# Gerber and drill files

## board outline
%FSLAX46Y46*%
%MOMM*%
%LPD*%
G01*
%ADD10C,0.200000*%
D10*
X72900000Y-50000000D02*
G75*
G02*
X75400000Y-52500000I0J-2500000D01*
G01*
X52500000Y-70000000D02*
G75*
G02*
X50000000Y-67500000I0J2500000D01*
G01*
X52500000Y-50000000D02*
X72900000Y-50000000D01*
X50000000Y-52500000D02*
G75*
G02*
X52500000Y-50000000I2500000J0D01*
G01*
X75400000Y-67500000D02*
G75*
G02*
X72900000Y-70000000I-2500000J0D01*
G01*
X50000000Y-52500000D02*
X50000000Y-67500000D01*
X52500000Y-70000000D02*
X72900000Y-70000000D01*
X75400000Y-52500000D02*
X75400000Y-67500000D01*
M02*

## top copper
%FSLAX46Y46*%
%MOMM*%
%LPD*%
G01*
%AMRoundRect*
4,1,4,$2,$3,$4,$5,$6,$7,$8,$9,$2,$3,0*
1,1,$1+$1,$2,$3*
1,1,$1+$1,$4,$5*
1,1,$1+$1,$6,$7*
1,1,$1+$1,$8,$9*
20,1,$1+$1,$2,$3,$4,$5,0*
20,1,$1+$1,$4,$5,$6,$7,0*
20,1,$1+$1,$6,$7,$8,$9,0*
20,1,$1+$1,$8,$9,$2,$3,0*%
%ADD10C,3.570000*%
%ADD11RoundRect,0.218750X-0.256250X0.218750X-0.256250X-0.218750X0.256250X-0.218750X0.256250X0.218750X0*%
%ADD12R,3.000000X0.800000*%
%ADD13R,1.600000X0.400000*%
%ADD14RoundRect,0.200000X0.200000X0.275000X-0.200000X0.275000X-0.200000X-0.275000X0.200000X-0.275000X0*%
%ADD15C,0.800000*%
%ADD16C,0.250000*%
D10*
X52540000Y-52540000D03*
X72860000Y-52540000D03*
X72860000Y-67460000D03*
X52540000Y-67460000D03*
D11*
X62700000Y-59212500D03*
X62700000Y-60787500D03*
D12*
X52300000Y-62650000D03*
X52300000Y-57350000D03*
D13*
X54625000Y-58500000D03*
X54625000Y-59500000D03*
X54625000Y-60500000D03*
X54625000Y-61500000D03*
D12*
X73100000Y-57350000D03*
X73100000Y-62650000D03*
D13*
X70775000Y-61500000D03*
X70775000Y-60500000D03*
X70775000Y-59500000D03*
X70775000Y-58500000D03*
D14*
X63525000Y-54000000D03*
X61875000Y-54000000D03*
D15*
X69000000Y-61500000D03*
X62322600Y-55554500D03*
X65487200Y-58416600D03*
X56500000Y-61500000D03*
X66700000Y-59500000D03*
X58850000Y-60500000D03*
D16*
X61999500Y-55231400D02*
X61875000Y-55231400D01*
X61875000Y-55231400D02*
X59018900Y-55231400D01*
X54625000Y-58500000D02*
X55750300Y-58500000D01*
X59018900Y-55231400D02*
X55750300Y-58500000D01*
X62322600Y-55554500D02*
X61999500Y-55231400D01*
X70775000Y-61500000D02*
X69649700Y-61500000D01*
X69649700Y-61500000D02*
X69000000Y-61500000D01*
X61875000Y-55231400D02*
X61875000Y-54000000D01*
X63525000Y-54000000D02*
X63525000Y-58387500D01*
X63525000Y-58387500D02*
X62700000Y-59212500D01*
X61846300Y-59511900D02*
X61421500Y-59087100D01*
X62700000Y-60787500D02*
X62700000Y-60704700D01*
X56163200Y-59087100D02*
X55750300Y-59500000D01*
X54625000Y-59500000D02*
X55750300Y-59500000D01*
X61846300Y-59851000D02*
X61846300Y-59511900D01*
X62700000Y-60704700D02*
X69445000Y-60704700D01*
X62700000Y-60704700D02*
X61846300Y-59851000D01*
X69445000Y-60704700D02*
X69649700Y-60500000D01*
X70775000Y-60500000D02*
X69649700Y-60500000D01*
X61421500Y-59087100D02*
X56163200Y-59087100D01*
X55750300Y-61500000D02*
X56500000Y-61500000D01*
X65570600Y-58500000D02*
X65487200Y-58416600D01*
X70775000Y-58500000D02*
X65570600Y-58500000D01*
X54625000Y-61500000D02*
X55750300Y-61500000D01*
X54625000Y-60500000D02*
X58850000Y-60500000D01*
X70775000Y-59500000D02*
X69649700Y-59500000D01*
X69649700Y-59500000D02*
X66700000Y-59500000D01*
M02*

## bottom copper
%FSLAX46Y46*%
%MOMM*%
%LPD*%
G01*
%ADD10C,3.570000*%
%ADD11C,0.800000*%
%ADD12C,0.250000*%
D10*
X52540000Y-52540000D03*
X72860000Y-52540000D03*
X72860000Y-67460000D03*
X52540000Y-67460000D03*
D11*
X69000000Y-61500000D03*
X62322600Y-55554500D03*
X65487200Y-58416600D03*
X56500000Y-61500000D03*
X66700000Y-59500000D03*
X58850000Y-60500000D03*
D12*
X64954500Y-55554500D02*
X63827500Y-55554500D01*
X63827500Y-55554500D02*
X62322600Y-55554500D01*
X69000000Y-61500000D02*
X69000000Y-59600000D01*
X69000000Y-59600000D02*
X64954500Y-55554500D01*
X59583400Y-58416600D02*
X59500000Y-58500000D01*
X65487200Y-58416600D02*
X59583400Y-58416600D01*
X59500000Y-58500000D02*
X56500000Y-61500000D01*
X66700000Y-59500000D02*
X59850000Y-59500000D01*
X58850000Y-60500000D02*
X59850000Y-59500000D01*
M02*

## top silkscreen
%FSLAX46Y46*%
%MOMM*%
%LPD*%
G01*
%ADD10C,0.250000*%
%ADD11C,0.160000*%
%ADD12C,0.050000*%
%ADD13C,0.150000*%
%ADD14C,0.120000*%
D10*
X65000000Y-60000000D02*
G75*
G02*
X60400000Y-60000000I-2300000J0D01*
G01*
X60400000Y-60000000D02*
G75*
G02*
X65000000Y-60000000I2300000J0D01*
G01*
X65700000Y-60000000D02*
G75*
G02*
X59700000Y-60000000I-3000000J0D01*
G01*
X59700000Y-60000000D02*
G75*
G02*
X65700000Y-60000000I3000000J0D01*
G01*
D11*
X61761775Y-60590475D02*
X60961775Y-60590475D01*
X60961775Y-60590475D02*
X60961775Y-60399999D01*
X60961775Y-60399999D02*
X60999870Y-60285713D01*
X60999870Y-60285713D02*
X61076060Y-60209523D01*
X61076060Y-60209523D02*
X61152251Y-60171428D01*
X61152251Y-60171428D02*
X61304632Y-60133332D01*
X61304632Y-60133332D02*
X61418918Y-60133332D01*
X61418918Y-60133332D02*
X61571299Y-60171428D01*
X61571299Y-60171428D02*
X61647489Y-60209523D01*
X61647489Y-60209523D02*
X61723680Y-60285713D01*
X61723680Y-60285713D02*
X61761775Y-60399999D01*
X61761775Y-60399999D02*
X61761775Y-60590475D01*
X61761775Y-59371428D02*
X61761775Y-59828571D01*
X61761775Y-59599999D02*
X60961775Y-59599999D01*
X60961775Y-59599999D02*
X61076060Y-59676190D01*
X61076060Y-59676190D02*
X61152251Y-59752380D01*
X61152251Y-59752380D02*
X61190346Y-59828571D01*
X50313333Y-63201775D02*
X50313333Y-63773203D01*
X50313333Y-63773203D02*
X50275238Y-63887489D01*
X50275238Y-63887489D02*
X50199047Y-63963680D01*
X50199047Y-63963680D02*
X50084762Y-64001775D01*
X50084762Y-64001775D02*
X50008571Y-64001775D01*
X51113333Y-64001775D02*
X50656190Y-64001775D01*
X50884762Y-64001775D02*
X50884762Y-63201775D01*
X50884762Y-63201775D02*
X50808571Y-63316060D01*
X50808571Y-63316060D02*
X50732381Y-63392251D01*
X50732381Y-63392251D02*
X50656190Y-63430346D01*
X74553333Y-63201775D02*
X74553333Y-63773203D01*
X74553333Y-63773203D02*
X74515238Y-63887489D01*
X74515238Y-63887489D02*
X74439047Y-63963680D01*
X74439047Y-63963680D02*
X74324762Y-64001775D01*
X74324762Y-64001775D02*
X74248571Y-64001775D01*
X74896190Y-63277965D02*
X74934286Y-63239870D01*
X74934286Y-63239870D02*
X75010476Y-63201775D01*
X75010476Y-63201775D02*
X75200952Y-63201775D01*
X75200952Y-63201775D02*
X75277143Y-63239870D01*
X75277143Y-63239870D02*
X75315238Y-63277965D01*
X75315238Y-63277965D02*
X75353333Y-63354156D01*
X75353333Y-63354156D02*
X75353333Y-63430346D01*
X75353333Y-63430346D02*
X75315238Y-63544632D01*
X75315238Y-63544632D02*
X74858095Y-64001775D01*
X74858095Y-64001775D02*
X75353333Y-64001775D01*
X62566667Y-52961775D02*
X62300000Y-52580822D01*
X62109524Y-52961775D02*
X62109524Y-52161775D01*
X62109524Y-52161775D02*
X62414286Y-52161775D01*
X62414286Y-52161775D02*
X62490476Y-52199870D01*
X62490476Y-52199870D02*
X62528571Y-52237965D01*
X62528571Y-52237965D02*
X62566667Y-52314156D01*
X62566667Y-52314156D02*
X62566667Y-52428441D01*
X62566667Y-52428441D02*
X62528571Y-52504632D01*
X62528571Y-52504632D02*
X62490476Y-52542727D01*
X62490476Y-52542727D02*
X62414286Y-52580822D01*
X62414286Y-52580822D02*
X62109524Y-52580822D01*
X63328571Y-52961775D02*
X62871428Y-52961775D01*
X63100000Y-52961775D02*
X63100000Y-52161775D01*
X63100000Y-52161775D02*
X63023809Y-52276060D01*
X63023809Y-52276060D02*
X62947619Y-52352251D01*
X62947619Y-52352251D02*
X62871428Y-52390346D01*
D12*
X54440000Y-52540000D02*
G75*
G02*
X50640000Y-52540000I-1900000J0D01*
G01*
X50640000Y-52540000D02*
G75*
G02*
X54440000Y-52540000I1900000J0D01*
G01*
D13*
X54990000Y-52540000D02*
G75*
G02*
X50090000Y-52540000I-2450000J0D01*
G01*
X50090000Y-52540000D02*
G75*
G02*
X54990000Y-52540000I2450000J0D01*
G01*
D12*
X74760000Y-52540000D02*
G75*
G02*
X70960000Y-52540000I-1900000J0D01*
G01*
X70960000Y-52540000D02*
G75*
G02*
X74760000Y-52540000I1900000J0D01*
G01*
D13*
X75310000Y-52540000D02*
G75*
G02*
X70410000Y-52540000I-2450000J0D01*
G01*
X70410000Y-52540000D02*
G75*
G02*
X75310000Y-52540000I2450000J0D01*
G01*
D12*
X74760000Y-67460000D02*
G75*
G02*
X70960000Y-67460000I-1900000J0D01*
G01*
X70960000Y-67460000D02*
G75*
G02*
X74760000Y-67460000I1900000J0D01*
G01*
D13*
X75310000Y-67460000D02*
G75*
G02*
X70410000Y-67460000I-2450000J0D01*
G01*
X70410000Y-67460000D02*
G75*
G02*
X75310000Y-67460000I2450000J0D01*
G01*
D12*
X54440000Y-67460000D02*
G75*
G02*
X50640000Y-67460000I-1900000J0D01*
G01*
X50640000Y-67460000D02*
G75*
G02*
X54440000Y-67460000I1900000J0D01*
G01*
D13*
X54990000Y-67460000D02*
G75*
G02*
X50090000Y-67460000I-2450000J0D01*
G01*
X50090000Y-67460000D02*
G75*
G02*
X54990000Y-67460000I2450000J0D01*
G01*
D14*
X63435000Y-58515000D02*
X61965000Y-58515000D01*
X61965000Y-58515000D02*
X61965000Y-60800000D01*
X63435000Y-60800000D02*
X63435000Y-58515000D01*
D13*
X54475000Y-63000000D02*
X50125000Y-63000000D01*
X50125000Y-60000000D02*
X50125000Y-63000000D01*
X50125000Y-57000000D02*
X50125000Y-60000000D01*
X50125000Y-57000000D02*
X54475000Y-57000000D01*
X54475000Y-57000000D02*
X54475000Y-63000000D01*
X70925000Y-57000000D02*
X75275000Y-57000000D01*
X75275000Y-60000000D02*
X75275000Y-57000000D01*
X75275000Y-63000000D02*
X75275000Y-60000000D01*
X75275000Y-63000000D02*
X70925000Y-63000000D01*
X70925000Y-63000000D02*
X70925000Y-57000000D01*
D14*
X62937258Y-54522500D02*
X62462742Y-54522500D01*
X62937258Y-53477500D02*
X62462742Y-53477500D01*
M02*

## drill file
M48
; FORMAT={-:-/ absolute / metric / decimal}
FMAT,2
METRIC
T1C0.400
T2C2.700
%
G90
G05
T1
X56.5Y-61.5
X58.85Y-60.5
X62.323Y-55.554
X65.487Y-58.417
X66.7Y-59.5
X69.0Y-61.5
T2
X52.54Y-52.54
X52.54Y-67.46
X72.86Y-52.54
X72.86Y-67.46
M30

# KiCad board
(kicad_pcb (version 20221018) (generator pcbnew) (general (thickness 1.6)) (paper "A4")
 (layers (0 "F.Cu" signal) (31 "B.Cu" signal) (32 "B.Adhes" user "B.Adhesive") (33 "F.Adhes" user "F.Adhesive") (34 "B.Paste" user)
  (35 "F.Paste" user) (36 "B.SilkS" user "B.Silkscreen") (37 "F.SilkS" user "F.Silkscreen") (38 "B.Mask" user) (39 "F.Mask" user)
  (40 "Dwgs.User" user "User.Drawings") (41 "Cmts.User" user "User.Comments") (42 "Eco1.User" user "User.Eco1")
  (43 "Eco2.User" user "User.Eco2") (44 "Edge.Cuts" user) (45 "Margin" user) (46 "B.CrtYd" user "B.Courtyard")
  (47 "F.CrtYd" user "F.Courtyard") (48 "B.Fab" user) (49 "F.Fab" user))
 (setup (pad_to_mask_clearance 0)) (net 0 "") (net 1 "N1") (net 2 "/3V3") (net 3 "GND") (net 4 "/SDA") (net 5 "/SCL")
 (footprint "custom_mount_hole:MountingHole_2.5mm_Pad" (layer "F.Cu") (at 52.54 52.54)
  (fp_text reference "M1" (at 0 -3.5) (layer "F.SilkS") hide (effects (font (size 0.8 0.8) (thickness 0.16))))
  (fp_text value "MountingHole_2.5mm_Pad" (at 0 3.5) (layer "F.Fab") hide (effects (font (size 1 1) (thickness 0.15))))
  (fp_circle (center 0 0) (end 1.9 0) (stroke (width 0.05) (type solid)) (fill none) (layer "F.SilkS"))
  (fp_circle (center 0 0) (end 2.45 0) (stroke (width 0.15) (type solid)) (fill none) (layer "F.SilkS"))
  (pad "~" thru_hole circle (at 0 0) (size 3.57 3.57) (drill 2.7) (layers "*.Cu" "*.Mask")))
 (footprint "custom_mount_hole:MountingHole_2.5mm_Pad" (layer "F.Cu") (at 72.86 52.54)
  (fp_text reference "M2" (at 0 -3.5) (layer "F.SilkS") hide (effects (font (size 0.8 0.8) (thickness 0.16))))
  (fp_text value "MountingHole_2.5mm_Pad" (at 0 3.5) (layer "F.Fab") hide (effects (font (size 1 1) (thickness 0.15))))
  (fp_circle (center 0 0) (end 1.9 0) (stroke (width 0.05) (type solid)) (fill none) (layer "F.SilkS"))
  (fp_circle (center 0 0) (end 2.45 0) (stroke (width 0.15) (type solid)) (fill none) (layer "F.SilkS"))
  (pad "~" thru_hole circle (at 0 0) (size 3.57 3.57) (drill 2.7) (layers "*.Cu" "*.Mask")))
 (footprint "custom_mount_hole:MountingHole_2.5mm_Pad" (layer "F.Cu") (at 72.86 67.46)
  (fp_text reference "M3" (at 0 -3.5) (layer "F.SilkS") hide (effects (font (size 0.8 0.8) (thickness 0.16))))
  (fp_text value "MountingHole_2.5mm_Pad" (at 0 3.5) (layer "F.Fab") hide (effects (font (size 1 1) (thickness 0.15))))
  (fp_circle (center 0 0) (end 1.9 0) (stroke (width 0.05) (type solid)) (fill none) (layer "F.SilkS"))
  (fp_circle (center 0 0) (end 2.45 0) (stroke (width 0.15) (type solid)) (fill none) (layer "F.SilkS"))
  (pad "~" thru_hole circle (at 0 0) (size 3.57 3.57) (drill 2.7) (layers "*.Cu" "*.Mask")))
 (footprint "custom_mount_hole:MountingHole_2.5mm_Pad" (layer "F.Cu") (at 52.54 67.46)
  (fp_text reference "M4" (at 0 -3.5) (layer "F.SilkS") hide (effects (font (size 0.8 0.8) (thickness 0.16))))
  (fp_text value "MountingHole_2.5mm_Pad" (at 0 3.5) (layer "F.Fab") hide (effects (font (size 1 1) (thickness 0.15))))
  (fp_circle (center 0 0) (end 1.9 0) (stroke (width 0.05) (type solid)) (fill none) (layer "F.SilkS"))
  (fp_circle (center 0 0) (end 2.45 0) (stroke (width 0.15) (type solid)) (fill none) (layer "F.SilkS"))
  (pad "~" thru_hole circle (at 0 0) (size 3.57 3.57) (drill 2.7) (layers "*.Cu" "*.Mask")))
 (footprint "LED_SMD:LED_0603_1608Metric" (layer "F.Cu") (at 62.7 60 -90)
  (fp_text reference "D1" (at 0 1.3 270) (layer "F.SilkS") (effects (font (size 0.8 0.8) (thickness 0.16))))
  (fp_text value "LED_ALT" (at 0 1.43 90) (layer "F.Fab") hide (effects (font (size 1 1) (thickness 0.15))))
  (fp_line (start -1.485 -0.735) (end -1.485 0.735) (stroke (width 0.12) (type solid)) (layer "F.SilkS"))
  (fp_line (start -1.485 0.735) (end 0.8 0.735) (stroke (width 0.12) (type solid)) (layer "F.SilkS"))
  (fp_line (start 0.8 -0.735) (end -1.485 -0.735) (stroke (width 0.12) (type solid)) (layer "F.SilkS"))
  (pad "1" smd roundrect (at -0.7875 0 270) (size 0.875 0.95) (layers "F.Cu" "F.Paste" "F.Mask") (roundrect_rratio 0.25) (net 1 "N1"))
  (pad "2" smd roundrect (at 0.7875 0 270) (size 0.875 0.95) (layers "F.Cu" "F.Paste" "F.Mask") (roundrect_rratio 0.25) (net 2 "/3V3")))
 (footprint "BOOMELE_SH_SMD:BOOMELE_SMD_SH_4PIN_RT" (layer "F.Cu") (at 52.78 60 90)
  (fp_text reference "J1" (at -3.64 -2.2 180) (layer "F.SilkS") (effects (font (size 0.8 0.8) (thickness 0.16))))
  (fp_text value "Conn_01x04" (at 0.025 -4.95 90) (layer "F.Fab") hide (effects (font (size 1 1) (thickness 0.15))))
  (fp_line (start -3 1.695) (end -3 -2.655) (stroke (width 0.15) (type solid)) (layer "F.SilkS"))
  (fp_line (start 0 -2.655) (end -3 -2.655) (stroke (width 0.15) (type solid)) (layer "F.SilkS"))
  (fp_line (start 3 -2.655) (end 0 -2.655) (stroke (width 0.15) (type solid)) (layer "F.SilkS"))
  (fp_line (start 3 -2.655) (end 3 1.695) (stroke (width 0.15) (type solid)) (layer "F.SilkS"))
  (fp_line (start 3 1.695) (end -3 1.695) (stroke (width 0.15) (type solid)) (layer "F.SilkS"))
  (pad "" smd rect (at -2.65 -0.48 270) (size 0.8 3) (layers "F.Cu" "F.Paste" "F.Mask"))
  (pad "" smd rect (at 2.65 -0.48 270) (size 0.8 3) (layers "F.Cu" "F.Paste" "F.Mask"))
  (pad "1" smd rect (at 1.5 1.845 270) (size 0.4 1.6) (layers "F.Cu" "F.Paste" "F.Mask") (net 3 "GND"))
  (pad "2" smd rect (at 0.5 1.845 270) (size 0.4 1.6) (layers "F.Cu" "F.Paste" "F.Mask") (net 2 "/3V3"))
  (pad "3" smd rect (at -0.5 1.845 270) (size 0.4 1.6) (layers "F.Cu" "F.Paste" "F.Mask") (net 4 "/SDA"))
  (pad "4" smd rect (at -1.5 1.845 270) (size 0.4 1.6) (layers "F.Cu" "F.Paste" "F.Mask") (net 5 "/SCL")))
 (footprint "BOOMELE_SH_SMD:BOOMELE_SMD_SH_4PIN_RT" (layer "F.Cu") (at 72.62 60 -90)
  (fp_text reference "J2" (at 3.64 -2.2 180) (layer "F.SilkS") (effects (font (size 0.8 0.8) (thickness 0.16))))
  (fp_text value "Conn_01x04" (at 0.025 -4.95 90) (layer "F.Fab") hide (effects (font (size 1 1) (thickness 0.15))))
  (fp_line (start -3 1.695) (end -3 -2.655) (stroke (width 0.15) (type solid)) (layer "F.SilkS"))
  (fp_line (start 0 -2.655) (end -3 -2.655) (stroke (width 0.15) (type solid)) (layer "F.SilkS"))
  (fp_line (start 3 -2.655) (end 0 -2.655) (stroke (width 0.15) (type solid)) (layer "F.SilkS"))
  (fp_line (start 3 -2.655) (end 3 1.695) (stroke (width 0.15) (type solid)) (layer "F.SilkS"))
  (fp_line (start 3 1.695) (end -3 1.695) (stroke (width 0.15) (type solid)) (layer "F.SilkS"))
  (pad "" smd rect (at -2.65 -0.48 90) (size 0.8 3) (layers "F.Cu" "F.Paste" "F.Mask"))
  (pad "" smd rect (at 2.65 -0.48 90) (size 0.8 3) (layers "F.Cu" "F.Paste" "F.Mask"))
  (pad "1" smd rect (at 1.5 1.845 90) (size 0.4 1.6) (layers "F.Cu" "F.Paste" "F.Mask") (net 3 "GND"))
  (pad "2" smd rect (at 0.5 1.845 90) (size 0.4 1.6) (layers "F.Cu" "F.Paste" "F.Mask") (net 2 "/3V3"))
  (pad "3" smd rect (at -0.5 1.845 90) (size 0.4 1.6) (layers "F.Cu" "F.Paste" "F.Mask") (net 4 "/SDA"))
  (pad "4" smd rect (at -1.5 1.845 90) (size 0.4 1.6) (layers "F.Cu" "F.Paste" "F.Mask") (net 5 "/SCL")))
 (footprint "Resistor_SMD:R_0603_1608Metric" (layer "F.Cu") (at 62.7 54 180)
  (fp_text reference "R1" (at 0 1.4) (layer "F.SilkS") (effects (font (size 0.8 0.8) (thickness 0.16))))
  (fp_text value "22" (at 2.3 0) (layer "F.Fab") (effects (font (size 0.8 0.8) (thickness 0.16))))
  (fp_line (start -0.237258 -0.5225) (end 0.237258 -0.5225) (stroke (width 0.12) (type solid)) (layer "F.SilkS"))
  (fp_line (start -0.237258 0.5225) (end 0.237258 0.5225) (stroke (width 0.12) (type solid)) (layer "F.SilkS"))
  (pad "1" smd roundrect (at -0.825 0 180) (size 0.8 0.95) (layers "F.Cu" "F.Paste" "F.Mask") (roundrect_rratio 0.25) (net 1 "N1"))
  (pad "2" smd roundrect (at 0.825 0 180) (size 0.8 0.95) (layers "F.Cu" "F.Paste" "F.Mask") (roundrect_rratio 0.25) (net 3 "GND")))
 (gr_circle (center 62.7 60) (end 65 60) (stroke (width 0.25) (type solid)) (fill none) (layer "F.SilkS"))
 (gr_circle (center 62.7 60) (end 65.7 60) (stroke (width 0.25) (type solid)) (fill none) (layer "F.SilkS"))
 (gr_arc (start 72.9 50) (mid 74.667767 50.732233) (end 75.4 52.5) (stroke (width 0.2) (type solid)) (layer "Edge.Cuts"))
 (gr_arc (start 52.5 70) (mid 50.732233 69.267767) (end 50 67.5) (stroke (width 0.2) (type solid)) (layer "Edge.Cuts"))
 (gr_line (start 52.5 50) (end 72.9 50) (stroke (width 0.2) (type solid)) (layer "Edge.Cuts"))
 (gr_arc (start 50 52.5) (mid 50.732233 50.732233) (end 52.5 50) (stroke (width 0.2) (type solid)) (layer "Edge.Cuts"))
 (gr_arc (start 75.4 67.5) (mid 74.667767 69.267767) (end 72.9 70) (stroke (width 0.2) (type solid)) (layer "Edge.Cuts"))
 (gr_line (start 50 52.5) (end 50 67.5) (stroke (width 0.2) (type solid)) (layer "Edge.Cuts"))
 (gr_line (start 52.5 70) (end 72.9 70) (stroke (width 0.2) (type solid)) (layer "Edge.Cuts"))
 (gr_line (start 75.4 52.5) (end 75.4 67.5) (stroke (width 0.2) (type solid)) (layer "Edge.Cuts"))
 (segment (start 61.9995 55.2314) (end 61.875 55.2314) (width 0.25) (layer "F.Cu") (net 3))
 (segment (start 61.875 55.2314) (end 59.0189 55.2314) (width 0.25) (layer "F.Cu") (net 3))
 (segment (start 54.625 58.5) (end 55.7503 58.5) (width 0.25) (layer "F.Cu") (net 3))
 (segment (start 59.0189 55.2314) (end 55.7503 58.5) (width 0.25) (layer "F.Cu") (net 3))
 (segment (start 62.3226 55.5545) (end 61.9995 55.2314) (width 0.25) (layer "F.Cu") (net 3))
 (segment (start 70.775 61.5) (end 69.6497 61.5) (width 0.25) (layer "F.Cu") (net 3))
 (segment (start 69.6497 61.5) (end 69 61.5) (width 0.25) (layer "F.Cu") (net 3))
 (segment (start 61.875 55.2314) (end 61.875 54) (width 0.25) (layer "F.Cu") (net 3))
 (via (at 69 61.5) (size 0.8) (drill 0.4) (layers "F.Cu" "B.Cu") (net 3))
 (via (at 62.3226 55.5545) (size 0.8) (drill 0.4) (layers "F.Cu" "B.Cu") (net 3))
 (segment (start 64.9545 55.5545) (end 63.8275 55.5545) (width 0.25) (layer "B.Cu") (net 3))
 (segment (start 63.8275 55.5545) (end 62.3226 55.5545) (width 0.25) (layer "B.Cu") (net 3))
 (segment (start 69 61.5) (end 69 59.6) (width 0.25) (layer "B.Cu") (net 3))
 (segment (start 69 59.6) (end 64.9545 55.5545) (width 0.25) (layer "B.Cu") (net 3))
 (segment (start 63.525 54) (end 63.525 58.3875) (width 0.25) (layer "F.Cu") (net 1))
 (segment (start 63.525 58.3875) (end 62.7 59.2125) (width 0.25) (layer "F.Cu") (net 1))
 (segment (start 61.8463 59.5119) (end 61.4215 59.0871) (width 0.25) (layer "F.Cu") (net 2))
 (segment (start 62.7 60.7875) (end 62.7 60.7047) (width 0.25) (layer "F.Cu") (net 2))
 (segment (start 56.1632 59.0871) (end 55.7503 59.5) (width 0.25) (layer "F.Cu") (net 2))
 (segment (start 54.625 59.5) (end 55.7503 59.5) (width 0.25) (layer "F.Cu") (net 2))
 (segment (start 61.8463 59.851) (end 61.8463 59.5119) (width 0.25) (layer "F.Cu") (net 2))
 (segment (start 62.7 60.7047) (end 69.445 60.7047) (width 0.25) (layer "F.Cu") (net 2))
 (segment (start 62.7 60.7047) (end 61.8463 59.851) (width 0.25) (layer "F.Cu") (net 2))
 (segment (start 69.445 60.7047) (end 69.6497 60.5) (width 0.25) (layer "F.Cu") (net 2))
 (segment (start 70.775 60.5) (end 69.6497 60.5) (width 0.25) (layer "F.Cu") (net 2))
 (segment (start 61.4215 59.0871) (end 56.1632 59.0871) (width 0.25) (layer "F.Cu") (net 2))
 (segment (start 55.7503 61.5) (end 56.5 61.5) (width 0.25) (layer "F.Cu") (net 5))
 (segment (start 65.5706 58.5) (end 65.4872 58.4166) (width 0.25) (layer "F.Cu") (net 5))
 (segment (start 70.775 58.5) (end 65.5706 58.5) (width 0.25) (layer "F.Cu") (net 5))
 (segment (start 54.625 61.5) (end 55.7503 61.5) (width 0.25) (layer "F.Cu") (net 5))
 (via (at 65.4872 58.4166) (size 0.8) (drill 0.4) (layers "F.Cu" "B.Cu") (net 5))
 (via (at 56.5 61.5) (size 0.8) (drill 0.4) (layers "F.Cu" "B.Cu") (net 5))
 (segment (start 59.5834 58.4166) (end 59.5 58.5) (width 0.25) (layer "B.Cu") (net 5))
 (segment (start 65.4872 58.4166) (end 59.5834 58.4166) (width 0.25) (layer "B.Cu") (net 5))
 (segment (start 59.5 58.5) (end 56.5 61.5) (width 0.25) (layer "B.Cu") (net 5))
 (segment (start 54.625 60.5) (end 58.85 60.5) (width 0.25) (layer "F.Cu") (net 4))
 (segment (start 70.775 59.5) (end 69.6497 59.5) (width 0.25) (layer "F.Cu") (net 4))
 (segment (start 69.6497 59.5) (end 66.7 59.5) (width 0.25) (layer "F.Cu") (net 4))
 (via (at 66.7 59.5) (size 0.8) (drill 0.4) (layers "F.Cu" "B.Cu") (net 4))
 (via (at 58.85 60.5) (size 0.8) (drill 0.4) (layers "F.Cu" "B.Cu") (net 4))
 (segment (start 66.7 59.5) (end 59.85 59.5) (width 0.25) (layer "B.Cu") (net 4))
 (segment (start 58.85 60.5) (end 59.85 59.5) (width 0.25) (layer "B.Cu") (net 4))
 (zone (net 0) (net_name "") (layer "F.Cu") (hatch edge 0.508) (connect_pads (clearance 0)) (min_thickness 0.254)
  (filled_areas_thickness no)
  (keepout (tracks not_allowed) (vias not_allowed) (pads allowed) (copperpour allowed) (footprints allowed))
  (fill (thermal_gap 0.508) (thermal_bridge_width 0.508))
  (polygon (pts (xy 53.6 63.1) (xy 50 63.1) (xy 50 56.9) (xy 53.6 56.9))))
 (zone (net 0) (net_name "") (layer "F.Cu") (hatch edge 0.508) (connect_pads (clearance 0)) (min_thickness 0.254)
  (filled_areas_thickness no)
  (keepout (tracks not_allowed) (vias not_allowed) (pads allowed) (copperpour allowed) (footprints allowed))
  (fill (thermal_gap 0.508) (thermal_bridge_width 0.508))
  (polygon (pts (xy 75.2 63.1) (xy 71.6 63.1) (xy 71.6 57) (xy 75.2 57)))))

